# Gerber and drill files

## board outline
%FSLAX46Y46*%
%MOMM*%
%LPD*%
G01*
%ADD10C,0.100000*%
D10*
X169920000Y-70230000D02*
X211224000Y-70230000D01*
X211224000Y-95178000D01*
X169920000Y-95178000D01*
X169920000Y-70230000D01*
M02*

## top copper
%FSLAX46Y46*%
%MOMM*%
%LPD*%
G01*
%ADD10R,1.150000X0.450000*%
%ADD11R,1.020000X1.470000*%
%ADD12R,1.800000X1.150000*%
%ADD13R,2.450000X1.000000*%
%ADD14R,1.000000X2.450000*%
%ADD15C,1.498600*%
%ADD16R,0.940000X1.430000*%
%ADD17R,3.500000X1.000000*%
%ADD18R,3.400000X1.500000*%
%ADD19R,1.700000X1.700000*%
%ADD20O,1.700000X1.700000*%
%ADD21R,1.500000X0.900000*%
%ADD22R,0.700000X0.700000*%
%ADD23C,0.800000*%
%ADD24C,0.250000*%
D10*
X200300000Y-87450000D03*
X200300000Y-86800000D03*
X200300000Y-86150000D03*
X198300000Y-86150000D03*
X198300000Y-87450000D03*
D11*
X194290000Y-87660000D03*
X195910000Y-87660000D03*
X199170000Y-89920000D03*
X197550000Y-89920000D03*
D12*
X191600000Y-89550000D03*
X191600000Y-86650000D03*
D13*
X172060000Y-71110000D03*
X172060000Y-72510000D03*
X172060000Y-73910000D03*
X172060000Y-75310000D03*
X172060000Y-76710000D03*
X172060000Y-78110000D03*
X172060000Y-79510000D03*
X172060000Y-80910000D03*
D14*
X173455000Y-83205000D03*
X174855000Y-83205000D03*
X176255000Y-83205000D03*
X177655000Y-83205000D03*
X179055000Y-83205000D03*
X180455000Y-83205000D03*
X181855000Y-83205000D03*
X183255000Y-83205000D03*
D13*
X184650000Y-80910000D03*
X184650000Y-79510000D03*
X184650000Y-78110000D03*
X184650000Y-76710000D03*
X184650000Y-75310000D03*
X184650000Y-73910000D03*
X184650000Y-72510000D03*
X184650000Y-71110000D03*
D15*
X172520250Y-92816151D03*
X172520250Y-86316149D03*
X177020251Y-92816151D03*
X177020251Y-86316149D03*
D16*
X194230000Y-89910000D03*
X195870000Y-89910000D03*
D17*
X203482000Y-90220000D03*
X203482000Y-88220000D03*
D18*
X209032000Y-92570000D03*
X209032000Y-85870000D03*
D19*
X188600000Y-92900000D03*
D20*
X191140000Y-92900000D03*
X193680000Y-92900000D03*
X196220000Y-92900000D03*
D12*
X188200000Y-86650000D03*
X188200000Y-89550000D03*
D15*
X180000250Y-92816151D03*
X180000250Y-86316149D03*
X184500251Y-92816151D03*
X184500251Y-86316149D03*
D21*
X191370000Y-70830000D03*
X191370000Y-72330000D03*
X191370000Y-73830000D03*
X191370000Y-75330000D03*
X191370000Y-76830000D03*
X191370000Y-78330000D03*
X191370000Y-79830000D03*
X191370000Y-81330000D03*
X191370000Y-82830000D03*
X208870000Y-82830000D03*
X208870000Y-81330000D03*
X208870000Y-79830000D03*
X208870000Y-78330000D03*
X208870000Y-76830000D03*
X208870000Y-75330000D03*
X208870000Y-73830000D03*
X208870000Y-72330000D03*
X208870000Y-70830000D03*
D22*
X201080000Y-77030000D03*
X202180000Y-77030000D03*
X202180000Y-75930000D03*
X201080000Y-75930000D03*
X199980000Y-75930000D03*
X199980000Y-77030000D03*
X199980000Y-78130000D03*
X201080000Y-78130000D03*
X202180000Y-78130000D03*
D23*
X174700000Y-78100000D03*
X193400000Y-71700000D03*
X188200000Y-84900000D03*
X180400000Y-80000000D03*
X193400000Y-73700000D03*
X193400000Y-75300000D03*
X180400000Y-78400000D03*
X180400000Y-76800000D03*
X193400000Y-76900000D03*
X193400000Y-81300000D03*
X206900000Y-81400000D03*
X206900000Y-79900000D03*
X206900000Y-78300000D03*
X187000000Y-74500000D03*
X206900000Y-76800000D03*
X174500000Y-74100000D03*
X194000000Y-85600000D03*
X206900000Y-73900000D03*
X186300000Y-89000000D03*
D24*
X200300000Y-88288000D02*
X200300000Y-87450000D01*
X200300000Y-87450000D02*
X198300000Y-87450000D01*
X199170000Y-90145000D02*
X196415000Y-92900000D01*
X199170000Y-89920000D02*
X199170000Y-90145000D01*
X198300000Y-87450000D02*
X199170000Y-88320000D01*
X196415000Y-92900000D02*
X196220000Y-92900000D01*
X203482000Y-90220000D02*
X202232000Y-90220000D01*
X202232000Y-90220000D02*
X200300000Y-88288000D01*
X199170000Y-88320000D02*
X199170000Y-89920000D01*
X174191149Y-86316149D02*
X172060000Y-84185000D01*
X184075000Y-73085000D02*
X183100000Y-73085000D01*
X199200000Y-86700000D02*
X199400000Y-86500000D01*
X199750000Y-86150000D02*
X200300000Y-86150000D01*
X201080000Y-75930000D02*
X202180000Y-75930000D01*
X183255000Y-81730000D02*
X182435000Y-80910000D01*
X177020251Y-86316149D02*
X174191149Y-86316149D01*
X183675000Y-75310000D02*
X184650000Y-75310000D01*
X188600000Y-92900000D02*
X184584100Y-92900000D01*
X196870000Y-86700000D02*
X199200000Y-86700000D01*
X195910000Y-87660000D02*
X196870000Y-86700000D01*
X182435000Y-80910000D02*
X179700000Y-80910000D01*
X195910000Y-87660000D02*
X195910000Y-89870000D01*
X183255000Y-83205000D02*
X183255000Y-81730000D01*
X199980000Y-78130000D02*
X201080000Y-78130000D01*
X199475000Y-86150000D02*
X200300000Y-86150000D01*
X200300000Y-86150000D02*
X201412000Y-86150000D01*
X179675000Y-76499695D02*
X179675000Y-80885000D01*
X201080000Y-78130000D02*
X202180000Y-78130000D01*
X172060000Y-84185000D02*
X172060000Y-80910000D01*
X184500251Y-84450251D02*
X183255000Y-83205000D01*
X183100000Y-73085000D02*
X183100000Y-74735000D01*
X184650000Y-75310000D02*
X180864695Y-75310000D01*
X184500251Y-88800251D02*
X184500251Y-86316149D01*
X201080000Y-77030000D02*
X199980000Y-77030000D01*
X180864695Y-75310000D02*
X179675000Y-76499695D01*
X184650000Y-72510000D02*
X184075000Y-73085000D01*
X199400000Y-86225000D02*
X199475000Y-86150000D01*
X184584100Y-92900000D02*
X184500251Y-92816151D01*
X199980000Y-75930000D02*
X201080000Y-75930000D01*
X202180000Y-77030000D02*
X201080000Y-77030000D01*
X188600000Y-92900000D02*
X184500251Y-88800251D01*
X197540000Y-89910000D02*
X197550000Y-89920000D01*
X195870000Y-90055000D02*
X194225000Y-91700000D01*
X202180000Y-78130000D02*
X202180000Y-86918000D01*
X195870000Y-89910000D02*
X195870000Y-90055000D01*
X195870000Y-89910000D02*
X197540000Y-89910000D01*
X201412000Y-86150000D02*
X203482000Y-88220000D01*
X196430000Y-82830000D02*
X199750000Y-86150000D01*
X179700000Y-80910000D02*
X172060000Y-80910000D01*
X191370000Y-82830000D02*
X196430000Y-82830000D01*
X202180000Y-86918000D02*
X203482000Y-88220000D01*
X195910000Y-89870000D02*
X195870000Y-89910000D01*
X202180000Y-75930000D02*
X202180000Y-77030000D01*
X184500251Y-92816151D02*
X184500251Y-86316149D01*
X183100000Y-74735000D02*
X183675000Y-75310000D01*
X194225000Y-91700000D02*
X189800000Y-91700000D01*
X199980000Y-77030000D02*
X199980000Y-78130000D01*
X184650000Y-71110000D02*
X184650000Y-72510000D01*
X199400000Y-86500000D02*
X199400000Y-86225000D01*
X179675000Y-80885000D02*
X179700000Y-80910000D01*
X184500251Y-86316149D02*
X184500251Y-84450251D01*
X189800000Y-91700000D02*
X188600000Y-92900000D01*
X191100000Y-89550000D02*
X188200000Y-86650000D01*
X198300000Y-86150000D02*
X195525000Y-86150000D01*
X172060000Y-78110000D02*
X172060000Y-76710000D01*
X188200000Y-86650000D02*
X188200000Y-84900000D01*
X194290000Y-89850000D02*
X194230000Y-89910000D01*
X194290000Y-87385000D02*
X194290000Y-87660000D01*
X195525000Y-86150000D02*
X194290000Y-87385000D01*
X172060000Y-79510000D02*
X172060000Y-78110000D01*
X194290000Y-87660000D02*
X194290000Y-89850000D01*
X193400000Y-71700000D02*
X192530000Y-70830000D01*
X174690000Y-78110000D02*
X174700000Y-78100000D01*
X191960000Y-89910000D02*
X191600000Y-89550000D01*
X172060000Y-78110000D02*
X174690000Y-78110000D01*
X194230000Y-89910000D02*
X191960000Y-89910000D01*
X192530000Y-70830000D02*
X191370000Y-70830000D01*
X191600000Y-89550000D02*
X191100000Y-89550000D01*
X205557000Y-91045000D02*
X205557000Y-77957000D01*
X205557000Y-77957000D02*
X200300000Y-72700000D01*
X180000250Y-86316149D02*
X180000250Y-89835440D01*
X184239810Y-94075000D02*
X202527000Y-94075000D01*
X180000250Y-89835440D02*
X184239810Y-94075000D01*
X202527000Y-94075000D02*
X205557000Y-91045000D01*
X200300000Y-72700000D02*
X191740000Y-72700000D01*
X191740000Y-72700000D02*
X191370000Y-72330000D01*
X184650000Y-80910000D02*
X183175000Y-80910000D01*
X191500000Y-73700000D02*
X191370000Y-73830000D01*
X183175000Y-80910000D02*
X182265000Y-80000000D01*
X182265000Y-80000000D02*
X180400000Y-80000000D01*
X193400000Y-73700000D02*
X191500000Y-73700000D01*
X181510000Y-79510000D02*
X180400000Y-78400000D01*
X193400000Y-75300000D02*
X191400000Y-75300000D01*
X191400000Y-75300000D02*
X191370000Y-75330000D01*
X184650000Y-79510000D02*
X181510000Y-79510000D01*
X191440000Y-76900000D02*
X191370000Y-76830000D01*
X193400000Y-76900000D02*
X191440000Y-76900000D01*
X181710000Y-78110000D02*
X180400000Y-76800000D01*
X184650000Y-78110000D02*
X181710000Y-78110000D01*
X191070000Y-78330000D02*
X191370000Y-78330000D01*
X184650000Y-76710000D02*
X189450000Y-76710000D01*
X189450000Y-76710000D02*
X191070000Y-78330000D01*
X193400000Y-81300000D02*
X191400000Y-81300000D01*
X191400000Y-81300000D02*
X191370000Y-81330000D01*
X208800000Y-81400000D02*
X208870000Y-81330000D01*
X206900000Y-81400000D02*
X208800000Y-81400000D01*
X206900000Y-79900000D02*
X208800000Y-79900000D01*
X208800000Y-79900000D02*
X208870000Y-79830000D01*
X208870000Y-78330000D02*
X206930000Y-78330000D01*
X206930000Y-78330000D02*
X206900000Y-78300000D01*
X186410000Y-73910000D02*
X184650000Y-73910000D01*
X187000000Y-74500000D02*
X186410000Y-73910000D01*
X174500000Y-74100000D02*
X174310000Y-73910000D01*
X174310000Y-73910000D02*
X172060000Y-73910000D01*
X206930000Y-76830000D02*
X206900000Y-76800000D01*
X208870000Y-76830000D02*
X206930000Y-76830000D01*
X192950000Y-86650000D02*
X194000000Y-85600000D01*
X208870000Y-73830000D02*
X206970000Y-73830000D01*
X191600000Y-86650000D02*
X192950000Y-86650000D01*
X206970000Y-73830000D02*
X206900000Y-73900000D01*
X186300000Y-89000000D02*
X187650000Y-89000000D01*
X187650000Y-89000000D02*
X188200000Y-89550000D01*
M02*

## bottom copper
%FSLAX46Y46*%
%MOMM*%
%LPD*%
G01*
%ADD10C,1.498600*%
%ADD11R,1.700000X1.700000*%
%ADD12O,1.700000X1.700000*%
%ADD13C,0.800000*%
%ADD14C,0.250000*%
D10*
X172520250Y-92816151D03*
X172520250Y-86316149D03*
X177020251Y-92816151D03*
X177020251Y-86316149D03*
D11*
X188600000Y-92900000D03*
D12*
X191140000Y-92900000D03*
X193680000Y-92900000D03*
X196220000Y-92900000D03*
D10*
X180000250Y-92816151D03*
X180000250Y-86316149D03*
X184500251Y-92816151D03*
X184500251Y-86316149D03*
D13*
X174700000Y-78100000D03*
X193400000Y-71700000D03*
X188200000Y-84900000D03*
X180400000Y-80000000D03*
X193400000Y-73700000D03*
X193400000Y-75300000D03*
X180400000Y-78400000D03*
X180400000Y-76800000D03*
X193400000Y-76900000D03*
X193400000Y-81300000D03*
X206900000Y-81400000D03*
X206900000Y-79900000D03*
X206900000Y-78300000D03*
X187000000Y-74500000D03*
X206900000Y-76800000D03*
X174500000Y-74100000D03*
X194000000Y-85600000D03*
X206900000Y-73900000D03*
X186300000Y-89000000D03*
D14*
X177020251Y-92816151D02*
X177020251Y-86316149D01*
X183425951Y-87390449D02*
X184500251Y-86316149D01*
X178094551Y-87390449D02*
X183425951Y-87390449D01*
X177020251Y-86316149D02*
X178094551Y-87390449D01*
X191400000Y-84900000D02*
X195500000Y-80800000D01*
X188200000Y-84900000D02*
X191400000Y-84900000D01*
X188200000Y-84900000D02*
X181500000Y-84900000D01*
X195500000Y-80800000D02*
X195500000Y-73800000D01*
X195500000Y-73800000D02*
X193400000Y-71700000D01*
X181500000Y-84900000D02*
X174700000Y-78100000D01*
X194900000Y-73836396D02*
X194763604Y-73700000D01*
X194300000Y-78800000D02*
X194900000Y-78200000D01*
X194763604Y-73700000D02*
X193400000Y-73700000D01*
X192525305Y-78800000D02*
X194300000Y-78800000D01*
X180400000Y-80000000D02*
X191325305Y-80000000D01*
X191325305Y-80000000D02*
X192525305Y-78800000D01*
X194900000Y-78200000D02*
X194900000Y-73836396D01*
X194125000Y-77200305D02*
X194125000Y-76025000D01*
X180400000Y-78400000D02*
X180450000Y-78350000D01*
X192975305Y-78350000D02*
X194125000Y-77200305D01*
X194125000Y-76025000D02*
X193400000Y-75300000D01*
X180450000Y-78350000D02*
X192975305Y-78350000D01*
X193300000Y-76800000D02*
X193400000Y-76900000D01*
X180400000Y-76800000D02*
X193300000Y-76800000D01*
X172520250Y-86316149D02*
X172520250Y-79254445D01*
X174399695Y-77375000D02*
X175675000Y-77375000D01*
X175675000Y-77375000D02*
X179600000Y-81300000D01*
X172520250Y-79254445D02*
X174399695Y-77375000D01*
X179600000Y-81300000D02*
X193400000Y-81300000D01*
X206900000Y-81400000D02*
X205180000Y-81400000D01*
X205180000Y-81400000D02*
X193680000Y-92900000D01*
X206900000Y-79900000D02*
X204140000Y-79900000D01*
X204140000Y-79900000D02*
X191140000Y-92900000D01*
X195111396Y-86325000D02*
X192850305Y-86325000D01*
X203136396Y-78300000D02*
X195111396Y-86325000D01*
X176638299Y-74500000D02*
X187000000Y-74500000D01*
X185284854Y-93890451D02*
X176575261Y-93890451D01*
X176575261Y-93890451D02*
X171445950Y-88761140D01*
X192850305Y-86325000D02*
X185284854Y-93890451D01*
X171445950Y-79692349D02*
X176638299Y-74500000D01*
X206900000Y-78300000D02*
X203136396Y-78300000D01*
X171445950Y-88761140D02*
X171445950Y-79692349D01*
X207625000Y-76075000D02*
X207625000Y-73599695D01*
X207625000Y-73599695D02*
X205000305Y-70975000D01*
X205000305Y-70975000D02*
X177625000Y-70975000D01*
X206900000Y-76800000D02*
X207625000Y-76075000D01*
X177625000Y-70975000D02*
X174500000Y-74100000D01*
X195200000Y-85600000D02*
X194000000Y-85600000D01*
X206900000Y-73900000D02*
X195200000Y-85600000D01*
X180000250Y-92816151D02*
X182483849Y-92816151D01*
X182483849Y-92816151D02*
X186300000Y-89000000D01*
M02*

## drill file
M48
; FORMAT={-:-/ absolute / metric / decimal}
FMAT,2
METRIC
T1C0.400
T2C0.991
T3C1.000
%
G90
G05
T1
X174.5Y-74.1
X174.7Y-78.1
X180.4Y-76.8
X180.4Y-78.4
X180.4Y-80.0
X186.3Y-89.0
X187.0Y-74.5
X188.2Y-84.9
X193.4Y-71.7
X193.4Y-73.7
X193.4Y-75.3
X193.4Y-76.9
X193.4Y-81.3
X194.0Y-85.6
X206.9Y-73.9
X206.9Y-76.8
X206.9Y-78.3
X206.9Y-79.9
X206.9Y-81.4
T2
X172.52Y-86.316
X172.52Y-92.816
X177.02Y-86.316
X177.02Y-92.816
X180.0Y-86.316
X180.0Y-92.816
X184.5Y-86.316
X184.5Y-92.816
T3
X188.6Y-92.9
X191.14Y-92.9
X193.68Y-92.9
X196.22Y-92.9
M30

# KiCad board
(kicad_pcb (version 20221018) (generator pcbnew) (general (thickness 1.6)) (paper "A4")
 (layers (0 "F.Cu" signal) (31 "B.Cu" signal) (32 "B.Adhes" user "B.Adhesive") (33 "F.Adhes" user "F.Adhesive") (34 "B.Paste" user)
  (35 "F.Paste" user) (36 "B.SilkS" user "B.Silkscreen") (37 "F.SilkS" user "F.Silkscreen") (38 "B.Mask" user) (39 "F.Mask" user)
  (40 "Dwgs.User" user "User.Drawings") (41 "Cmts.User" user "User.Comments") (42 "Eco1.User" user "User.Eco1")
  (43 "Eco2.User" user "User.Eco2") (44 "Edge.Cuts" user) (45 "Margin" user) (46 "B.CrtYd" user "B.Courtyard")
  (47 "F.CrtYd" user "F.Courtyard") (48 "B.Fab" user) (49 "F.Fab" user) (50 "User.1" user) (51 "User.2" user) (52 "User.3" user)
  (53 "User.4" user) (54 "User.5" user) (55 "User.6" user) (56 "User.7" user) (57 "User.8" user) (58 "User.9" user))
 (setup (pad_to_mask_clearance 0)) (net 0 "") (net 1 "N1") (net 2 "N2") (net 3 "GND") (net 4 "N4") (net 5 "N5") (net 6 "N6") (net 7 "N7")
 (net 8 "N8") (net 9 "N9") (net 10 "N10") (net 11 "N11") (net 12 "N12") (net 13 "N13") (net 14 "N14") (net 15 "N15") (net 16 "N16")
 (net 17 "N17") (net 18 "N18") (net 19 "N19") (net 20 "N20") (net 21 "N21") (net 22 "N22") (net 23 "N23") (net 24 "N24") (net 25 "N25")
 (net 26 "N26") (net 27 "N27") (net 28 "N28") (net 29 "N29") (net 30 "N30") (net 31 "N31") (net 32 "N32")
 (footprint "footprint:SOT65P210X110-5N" (layer "F.Cu") (at 199.3 86.8 180)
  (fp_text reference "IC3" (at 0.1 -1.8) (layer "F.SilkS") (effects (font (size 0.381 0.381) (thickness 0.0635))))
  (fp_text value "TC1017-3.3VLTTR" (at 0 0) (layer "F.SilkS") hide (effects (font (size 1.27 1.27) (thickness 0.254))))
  (pad "1" smd rect (at -1 -0.65 270) (size 0.45 1.15) (layers "F.Cu" "F.Paste" "F.Mask") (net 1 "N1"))
  (pad "2" smd rect (at -1 0 270) (size 0.45 1.15) (layers "F.Cu" "F.Paste" "F.Mask") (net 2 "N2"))
  (pad "3" smd rect (at -1 0.65 270) (size 0.45 1.15) (layers "F.Cu" "F.Paste" "F.Mask") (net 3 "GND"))
  (pad "4" smd rect (at 1 0.65 270) (size 0.45 1.15) (layers "F.Cu" "F.Paste" "F.Mask") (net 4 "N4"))
  (pad "5" smd rect (at 1 -0.65 270) (size 0.45 1.15) (layers "F.Cu" "F.Paste" "F.Mask") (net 1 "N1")))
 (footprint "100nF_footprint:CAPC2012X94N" (layer "F.Cu") (at 195.1 87.66)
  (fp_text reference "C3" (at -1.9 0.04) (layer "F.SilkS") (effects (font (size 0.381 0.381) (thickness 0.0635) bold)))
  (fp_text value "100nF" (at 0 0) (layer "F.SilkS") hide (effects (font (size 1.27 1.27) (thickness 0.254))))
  (pad "1" smd rect (at -0.81 0) (size 1.02 1.47) (layers "F.Cu" "F.Paste" "F.Mask") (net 4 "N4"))
  (pad "2" smd rect (at 0.81 0) (size 1.02 1.47) (layers "F.Cu" "F.Paste" "F.Mask") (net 3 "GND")))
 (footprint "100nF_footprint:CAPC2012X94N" (layer "F.Cu") (at 198.36 89.92 180)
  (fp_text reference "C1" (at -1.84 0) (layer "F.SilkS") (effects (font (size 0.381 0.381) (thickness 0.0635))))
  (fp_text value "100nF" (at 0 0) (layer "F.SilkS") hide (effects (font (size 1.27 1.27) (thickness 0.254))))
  (pad "1" smd rect (at -0.81 0 180) (size 1.02 1.47) (layers "F.Cu" "F.Paste" "F.Mask") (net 1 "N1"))
  (pad "2" smd rect (at 0.81 0 180) (size 1.02 1.47) (layers "F.Cu" "F.Paste" "F.Mask") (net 3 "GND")))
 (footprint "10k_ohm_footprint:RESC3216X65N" (layer "F.Cu") (at 191.6 88.1 90)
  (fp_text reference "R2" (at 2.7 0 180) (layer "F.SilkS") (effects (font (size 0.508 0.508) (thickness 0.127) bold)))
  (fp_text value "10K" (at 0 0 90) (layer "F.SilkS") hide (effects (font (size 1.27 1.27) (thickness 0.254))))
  (pad "1" smd rect (at -1.45 0 90) (size 1.15 1.8) (layers "F.Cu" "F.Paste" "F.Mask") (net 4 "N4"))
  (pad "2" smd rect (at 1.45 0 90) (size 1.15 1.8) (layers "F.Cu" "F.Paste" "F.Mask") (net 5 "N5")))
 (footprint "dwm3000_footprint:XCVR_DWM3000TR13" (layer "F.Cu") (at 178.355 72.06)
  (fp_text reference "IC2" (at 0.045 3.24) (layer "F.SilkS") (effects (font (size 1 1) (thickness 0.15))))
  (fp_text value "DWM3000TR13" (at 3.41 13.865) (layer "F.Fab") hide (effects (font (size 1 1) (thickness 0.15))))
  (pad "1" smd rect (at -6.295 -0.95) (size 2.45 1) (layers "F.Cu" "F.Paste" "F.Mask") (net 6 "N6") (solder_mask_margin 0.102))
  (pad "2" smd rect (at -6.295 0.45) (size 2.45 1) (layers "F.Cu" "F.Paste" "F.Mask") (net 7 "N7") (solder_mask_margin 0.102))
  (pad "3" smd rect (at -6.295 1.85) (size 2.45 1) (layers "F.Cu" "F.Paste" "F.Mask") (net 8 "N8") (solder_mask_margin 0.102))
  (pad "4" smd rect (at -6.295 3.25) (size 2.45 1) (layers "F.Cu" "F.Paste" "F.Mask") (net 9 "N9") (solder_mask_margin 0.102))
  (pad "5" smd rect (at -6.295 4.65) (size 2.45 1) (layers "F.Cu" "F.Paste" "F.Mask") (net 4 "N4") (solder_mask_margin 0.102))
  (pad "6" smd rect (at -6.295 6.05) (size 2.45 1) (layers "F.Cu" "F.Paste" "F.Mask") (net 4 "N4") (solder_mask_margin 0.102))
  (pad "7" smd rect (at -6.295 7.45) (size 2.45 1) (layers "F.Cu" "F.Paste" "F.Mask") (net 4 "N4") (solder_mask_margin 0.102))
  (pad "8" smd rect (at -6.295 8.85) (size 2.45 1) (layers "F.Cu" "F.Paste" "F.Mask") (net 3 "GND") (solder_mask_margin 0.102))
  (pad "9" smd rect (at -4.9 11.145) (size 1 2.45) (layers "F.Cu" "F.Paste" "F.Mask") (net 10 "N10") (solder_mask_margin 0.102))
  (pad "10" smd rect (at -3.5 11.145) (size 1 2.45) (layers "F.Cu" "F.Paste" "F.Mask") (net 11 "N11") (solder_mask_margin 0.102))
  (pad "11" smd rect (at -2.1 11.145) (size 1 2.45) (layers "F.Cu" "F.Paste" "F.Mask") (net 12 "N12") (solder_mask_margin 0.102))
  (pad "12" smd rect (at -0.7 11.145) (size 1 2.45) (layers "F.Cu" "F.Paste" "F.Mask") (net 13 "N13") (solder_mask_margin 0.102))
  (pad "13" smd rect (at 0.7 11.145) (size 1 2.45) (layers "F.Cu" "F.Paste" "F.Mask") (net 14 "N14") (solder_mask_margin 0.102))
  (pad "14" smd rect (at 2.1 11.145) (size 1 2.45) (layers "F.Cu" "F.Paste" "F.Mask") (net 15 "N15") (solder_mask_margin 0.102))
  (pad "15" smd rect (at 3.5 11.145) (size 1 2.45) (layers "F.Cu" "F.Paste" "F.Mask") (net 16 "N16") (solder_mask_margin 0.102))
  (pad "16" smd rect (at 4.9 11.145) (size 1 2.45) (layers "F.Cu" "F.Paste" "F.Mask") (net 3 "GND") (solder_mask_margin 0.102))
  (pad "17" smd rect (at 6.295 8.85) (size 2.45 1) (layers "F.Cu" "F.Paste" "F.Mask") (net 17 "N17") (solder_mask_margin 0.102))
  (pad "18" smd rect (at 6.295 7.45) (size 2.45 1) (layers "F.Cu" "F.Paste" "F.Mask") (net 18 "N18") (solder_mask_margin 0.102))
  (pad "19" smd rect (at 6.295 6.05) (size 2.45 1) (layers "F.Cu" "F.Paste" "F.Mask") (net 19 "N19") (solder_mask_margin 0.102))
  (pad "20" smd rect (at 6.295 4.65) (size 2.45 1) (layers "F.Cu" "F.Paste" "F.Mask") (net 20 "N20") (solder_mask_margin 0.102))
  (pad "21" smd rect (at 6.295 3.25) (size 2.45 1) (layers "F.Cu" "F.Paste" "F.Mask") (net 3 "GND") (solder_mask_margin 0.102))
  (pad "22" smd rect (at 6.295 1.85) (size 2.45 1) (layers "F.Cu" "F.Paste" "F.Mask") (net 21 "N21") (solder_mask_margin 0.102))
  (pad "23" smd rect (at 6.295 0.45) (size 2.45 1) (layers "F.Cu" "F.Paste" "F.Mask") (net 3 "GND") (solder_mask_margin 0.102))
  (pad "24" smd rect (at 6.295 -0.95) (size 2.45 1) (layers "F.Cu" "F.Paste" "F.Mask") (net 3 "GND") (solder_mask_margin 0.102))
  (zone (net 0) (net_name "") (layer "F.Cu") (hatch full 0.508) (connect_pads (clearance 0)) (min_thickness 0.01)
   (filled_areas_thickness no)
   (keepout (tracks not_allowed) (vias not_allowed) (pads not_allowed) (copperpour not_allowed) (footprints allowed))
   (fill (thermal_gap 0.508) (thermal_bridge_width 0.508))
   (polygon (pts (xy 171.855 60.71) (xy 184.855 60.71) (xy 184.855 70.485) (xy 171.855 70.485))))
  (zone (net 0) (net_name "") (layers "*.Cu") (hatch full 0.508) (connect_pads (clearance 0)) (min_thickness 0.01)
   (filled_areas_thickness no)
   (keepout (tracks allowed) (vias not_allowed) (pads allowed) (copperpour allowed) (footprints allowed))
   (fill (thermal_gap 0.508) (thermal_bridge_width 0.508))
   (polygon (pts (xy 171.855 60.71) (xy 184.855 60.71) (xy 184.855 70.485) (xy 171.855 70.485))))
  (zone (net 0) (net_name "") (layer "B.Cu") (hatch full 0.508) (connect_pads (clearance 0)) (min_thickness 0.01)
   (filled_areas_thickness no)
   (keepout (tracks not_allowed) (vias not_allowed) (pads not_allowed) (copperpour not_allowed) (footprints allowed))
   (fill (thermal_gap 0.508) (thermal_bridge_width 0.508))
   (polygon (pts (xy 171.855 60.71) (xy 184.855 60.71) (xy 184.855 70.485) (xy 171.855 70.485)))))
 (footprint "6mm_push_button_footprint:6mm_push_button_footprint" (layer "F.Cu") (at 172.52025 92.816151 90)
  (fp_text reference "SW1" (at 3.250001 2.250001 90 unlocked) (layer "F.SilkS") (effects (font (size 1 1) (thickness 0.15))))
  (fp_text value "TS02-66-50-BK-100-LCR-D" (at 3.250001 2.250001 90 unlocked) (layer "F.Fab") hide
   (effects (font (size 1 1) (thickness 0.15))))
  (pad "1" thru_hole circle (at 0 0 90) (size 1.4986 1.4986) (drill 0.9906) (layers "*.Cu" "*.Mask") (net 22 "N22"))
  (pad "2" thru_hole circle (at 6.500002 0 90) (size 1.4986 1.4986) (drill 0.9906) (layers "*.Cu" "*.Mask") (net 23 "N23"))
  (pad "3" thru_hole circle (at 0 4.500001 90) (size 1.4986 1.4986) (drill 0.9906) (layers "*.Cu" "*.Mask") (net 3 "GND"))
  (pad "4" thru_hole circle (at 6.500002 4.500001 90) (size 1.4986 1.4986) (drill 0.9906) (layers "*.Cu" "*.Mask") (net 3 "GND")))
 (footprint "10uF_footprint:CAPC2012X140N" (layer "F.Cu") (at 195.05 89.91)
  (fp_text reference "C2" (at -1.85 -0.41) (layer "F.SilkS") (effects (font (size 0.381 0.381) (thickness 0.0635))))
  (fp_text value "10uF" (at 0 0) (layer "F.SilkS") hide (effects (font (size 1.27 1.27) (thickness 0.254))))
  (pad "1" smd rect (at -0.82 0) (size 0.94 1.43) (layers "F.Cu" "F.Paste" "F.Mask") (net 4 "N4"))
  (pad "2" smd rect (at 0.82 0) (size 0.94 1.43) (layers "F.Cu" "F.Paste" "F.Mask") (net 3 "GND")))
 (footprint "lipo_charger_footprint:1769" (layer "F.Cu") (at 203.482 89.22 90)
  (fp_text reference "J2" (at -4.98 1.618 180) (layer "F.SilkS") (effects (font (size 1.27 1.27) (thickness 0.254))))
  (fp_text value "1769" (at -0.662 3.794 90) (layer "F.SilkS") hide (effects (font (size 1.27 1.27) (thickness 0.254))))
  (pad "1" smd rect (at -1 0 90) (size 1 3.5) (layers "F.Cu" "F.Paste" "F.Mask") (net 1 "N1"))
  (pad "2" smd rect (at 1 0 90) (size 1 3.5) (layers "F.Cu" "F.Paste" "F.Mask") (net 3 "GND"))
  (pad "3" smd rect (at -3.35 5.55 90) (size 1.5 3.4) (layers "F.Cu" "F.Paste" "F.Mask"))
  (pad "4" smd rect (at 3.35 5.55 90) (size 1.5 3.4) (layers "F.Cu" "F.Paste" "F.Mask")))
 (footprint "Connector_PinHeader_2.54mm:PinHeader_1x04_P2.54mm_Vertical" (layer "F.Cu") (at 188.6 92.9 90)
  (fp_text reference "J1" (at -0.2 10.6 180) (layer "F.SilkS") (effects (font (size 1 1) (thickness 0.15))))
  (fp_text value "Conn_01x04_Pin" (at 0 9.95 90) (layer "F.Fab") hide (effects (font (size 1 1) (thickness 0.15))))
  (pad "1" thru_hole rect (at 0 0 90) (size 1.7 1.7) (drill 1) (layers "*.Cu" "*.Mask") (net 3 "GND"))
  (pad "2" thru_hole oval (at 0 2.54 90) (size 1.7 1.7) (drill 1) (layers "*.Cu" "*.Mask") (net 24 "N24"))
  (pad "3" thru_hole oval (at 0 5.08 90) (size 1.7 1.7) (drill 1) (layers "*.Cu" "*.Mask") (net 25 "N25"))
  (pad "4" thru_hole oval (at 0 7.62 90) (size 1.7 1.7) (drill 1) (layers "*.Cu" "*.Mask") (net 1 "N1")))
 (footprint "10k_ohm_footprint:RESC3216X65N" (layer "F.Cu") (at 188.2 88.1 -90)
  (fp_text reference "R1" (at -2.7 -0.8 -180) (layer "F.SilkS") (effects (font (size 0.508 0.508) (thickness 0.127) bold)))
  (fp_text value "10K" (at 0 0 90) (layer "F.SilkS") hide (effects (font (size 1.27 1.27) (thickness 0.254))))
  (pad "1" smd rect (at -1.45 0 270) (size 1.15 1.8) (layers "F.Cu" "F.Paste" "F.Mask") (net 4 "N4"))
  (pad "2" smd rect (at 1.45 0 270) (size 1.15 1.8) (layers "F.Cu" "F.Paste" "F.Mask") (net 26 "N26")))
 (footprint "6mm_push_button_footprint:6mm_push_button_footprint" (layer "F.Cu") (at 180.00025 92.816151 90)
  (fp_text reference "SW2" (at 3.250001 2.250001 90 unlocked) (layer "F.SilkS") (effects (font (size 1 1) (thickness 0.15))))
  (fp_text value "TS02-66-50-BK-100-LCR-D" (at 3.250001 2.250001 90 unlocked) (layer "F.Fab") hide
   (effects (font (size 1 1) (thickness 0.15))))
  (pad "1" thru_hole circle (at 0 0 90) (size 1.4986 1.4986) (drill 0.9906) (layers "*.Cu" "*.Mask") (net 26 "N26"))
  (pad "2" thru_hole circle (at 6.500002 0 90) (size 1.4986 1.4986) (drill 0.9906) (layers "*.Cu" "*.Mask") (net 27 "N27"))
  (pad "3" thru_hole circle (at 0 4.500001 90) (size 1.4986 1.4986) (drill 0.9906) (layers "*.Cu" "*.Mask") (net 3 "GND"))
  (pad "4" thru_hole circle (at 6.500002 4.500001 90) (size 1.4986 1.4986) (drill 0.9906) (layers "*.Cu" "*.Mask") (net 3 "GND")))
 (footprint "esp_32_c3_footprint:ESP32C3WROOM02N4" (layer "F.Cu") (at 201.08 77.03)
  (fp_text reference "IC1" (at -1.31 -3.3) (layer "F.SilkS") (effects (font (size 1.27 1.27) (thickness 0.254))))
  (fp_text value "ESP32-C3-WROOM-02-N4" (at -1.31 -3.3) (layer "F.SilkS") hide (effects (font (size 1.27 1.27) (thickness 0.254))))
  (pad "1" smd rect (at -9.71 -6.2 90) (size 0.9 1.5) (layers "F.Cu" "F.Paste" "F.Mask") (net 4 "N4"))
  (pad "2" smd rect (at -9.71 -4.7 90) (size 0.9 1.5) (layers "F.Cu" "F.Paste" "F.Mask") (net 27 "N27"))
  (pad "3" smd rect (at -9.71 -3.2 90) (size 0.9 1.5) (layers "F.Cu" "F.Paste" "F.Mask") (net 17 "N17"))
  (pad "4" smd rect (at -9.71 -1.7 90) (size 0.9 1.5) (layers "F.Cu" "F.Paste" "F.Mask") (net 18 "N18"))
  (pad "5" smd rect (at -9.71 -0.2 90) (size 0.9 1.5) (layers "F.Cu" "F.Paste" "F.Mask") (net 19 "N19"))
  (pad "6" smd rect (at -9.71 1.3 90) (size 0.9 1.5) (layers "F.Cu" "F.Paste" "F.Mask") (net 20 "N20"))
  (pad "7" smd rect (at -9.71 2.8 90) (size 0.9 1.5) (layers "F.Cu" "F.Paste" "F.Mask") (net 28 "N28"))
  (pad "8" smd rect (at -9.71 4.3 90) (size 0.9 1.5) (layers "F.Cu" "F.Paste" "F.Mask") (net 23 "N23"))
  (pad "9" smd rect (at -9.71 5.8 90) (size 0.9 1.5) (layers "F.Cu" "F.Paste" "F.Mask") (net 3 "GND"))
  (pad "10" smd rect (at 7.79 5.8 90) (size 0.9 1.5) (layers "F.Cu" "F.Paste" "F.Mask") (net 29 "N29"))
  (pad "11" smd rect (at 7.79 4.3 90) (size 0.9 1.5) (layers "F.Cu" "F.Paste" "F.Mask") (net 25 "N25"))
  (pad "12" smd rect (at 7.79 2.8 90) (size 0.9 1.5) (layers "F.Cu" "F.Paste" "F.Mask") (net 24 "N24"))
  (pad "13" smd rect (at 7.79 1.3 90) (size 0.9 1.5) (layers "F.Cu" "F.Paste" "F.Mask") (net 21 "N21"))
  (pad "14" smd rect (at 7.79 -0.2 90) (size 0.9 1.5) (layers "F.Cu" "F.Paste" "F.Mask") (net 8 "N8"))
  (pad "15" smd rect (at 7.79 -1.7 90) (size 0.9 1.5) (layers "F.Cu" "F.Paste" "F.Mask") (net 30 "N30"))
  (pad "16" smd rect (at 7.79 -3.2 90) (size 0.9 1.5) (layers "F.Cu" "F.Paste" "F.Mask") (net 5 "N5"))
  (pad "17" smd rect (at 7.79 -4.7 90) (size 0.9 1.5) (layers "F.Cu" "F.Paste" "F.Mask") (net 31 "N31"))
  (pad "18" smd rect (at 7.79 -6.2 90) (size 0.9 1.5) (layers "F.Cu" "F.Paste" "F.Mask") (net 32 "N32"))
  (pad "19" smd rect (at 0 0 90) (size 0.7 0.7) (layers "F.Cu" "F.Paste" "F.Mask") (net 3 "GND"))
  (pad "20" smd rect (at 1.1 0 90) (size 0.7 0.7) (layers "F.Cu" "F.Paste" "F.Mask") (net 3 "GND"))
  (pad "21" smd rect (at 1.1 -1.1 90) (size 0.7 0.7) (layers "F.Cu" "F.Paste" "F.Mask") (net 3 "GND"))
  (pad "22" smd rect (at 0 -1.1 90) (size 0.7 0.7) (layers "F.Cu" "F.Paste" "F.Mask") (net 3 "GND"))
  (pad "23" smd rect (at -1.1 -1.1 90) (size 0.7 0.7) (layers "F.Cu" "F.Paste" "F.Mask") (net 3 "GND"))
  (pad "24" smd rect (at -1.1 0 90) (size 0.7 0.7) (layers "F.Cu" "F.Paste" "F.Mask") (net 3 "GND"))
  (pad "25" smd rect (at -1.1 1.1 90) (size 0.7 0.7) (layers "F.Cu" "F.Paste" "F.Mask") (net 3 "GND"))
  (pad "26" smd rect (at 0 1.1 90) (size 0.7 0.7) (layers "F.Cu" "F.Paste" "F.Mask") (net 3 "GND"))
  (pad "27" smd rect (at 1.1 1.1 90) (size 0.7 0.7) (layers "F.Cu" "F.Paste" "F.Mask") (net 3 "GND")))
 (gr_rect (start 169.92 70.23) (end 211.224 95.178) (stroke (width 0.1) (type default)) (fill none) (layer "Edge.Cuts"))
 (segment (start 200.3 88.288) (end 200.3 87.45) (width 0.25) (layer "F.Cu") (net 1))
 (segment (start 200.3 87.45) (end 198.3 87.45) (width 0.25) (layer "F.Cu") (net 1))
 (segment (start 199.17 90.145) (end 196.415 92.9) (width 0.25) (layer "F.Cu") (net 1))
 (segment (start 199.17 89.92) (end 199.17 90.145) (width 0.25) (layer "F.Cu") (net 1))
 (segment (start 198.3 87.45) (end 199.17 88.32) (width 0.25) (layer "F.Cu") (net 1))
 (segment (start 196.415 92.9) (end 196.22 92.9) (width 0.25) (layer "F.Cu") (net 1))
 (segment (start 203.482 90.22) (end 202.232 90.22) (width 0.25) (layer "F.Cu") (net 1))
 (segment (start 202.232 90.22) (end 200.3 88.288) (width 0.25) (layer "F.Cu") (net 1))
 (segment (start 199.17 88.32) (end 199.17 89.92) (width 0.25) (layer "F.Cu") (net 1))
 (segment (start 174.191149 86.316149) (end 172.06 84.185) (width 0.25) (layer "F.Cu") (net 3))
 (segment (start 184.075 73.085) (end 183.1 73.085) (width 0.25) (layer "F.Cu") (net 3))
 (segment (start 199.2 86.7) (end 199.4 86.5) (width 0.25) (layer "F.Cu") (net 3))
 (segment (start 199.75 86.15) (end 200.3 86.15) (width 0.25) (layer "F.Cu") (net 3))
 (segment (start 201.08 75.93) (end 202.18 75.93) (width 0.25) (layer "F.Cu") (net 3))
 (segment (start 183.255 81.73) (end 182.435 80.91) (width 0.25) (layer "F.Cu") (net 3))
 (segment (start 177.020251 86.316149) (end 174.191149 86.316149) (width 0.25) (layer "F.Cu") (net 3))
 (segment (start 183.675 75.31) (end 184.65 75.31) (width 0.25) (layer "F.Cu") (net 3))
 (segment (start 188.6 92.9) (end 184.5841 92.9) (width 0.25) (layer "F.Cu") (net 3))
 (segment (start 196.87 86.7) (end 199.2 86.7) (width 0.25) (layer "F.Cu") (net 3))
 (segment (start 195.91 87.66) (end 196.87 86.7) (width 0.25) (layer "F.Cu") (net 3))
 (segment (start 182.435 80.91) (end 179.7 80.91) (width 0.25) (layer "F.Cu") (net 3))
 (segment (start 195.91 87.66) (end 195.91 89.87) (width 0.25) (layer "F.Cu") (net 3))
 (segment (start 183.255 83.205) (end 183.255 81.73) (width 0.25) (layer "F.Cu") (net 3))
 (segment (start 199.98 78.13) (end 201.08 78.13) (width 0.25) (layer "F.Cu") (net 3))
 (segment (start 199.475 86.15) (end 200.3 86.15) (width 0.25) (layer "F.Cu") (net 3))
 (segment (start 200.3 86.15) (end 201.412 86.15) (width 0.25) (layer "F.Cu") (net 3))
 (segment (start 179.675 76.499695) (end 179.675 80.885) (width 0.25) (layer "F.Cu") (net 3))
 (segment (start 201.08 78.13) (end 202.18 78.13) (width 0.25) (layer "F.Cu") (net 3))
 (segment (start 172.06 84.185) (end 172.06 80.91) (width 0.25) (layer "F.Cu") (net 3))
 (segment (start 184.500251 84.450251) (end 183.255 83.205) (width 0.25) (layer "F.Cu") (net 3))
 (segment (start 183.1 73.085) (end 183.1 74.735) (width 0.25) (layer "F.Cu") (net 3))
 (segment (start 184.65 75.31) (end 180.864695 75.31) (width 0.25) (layer "F.Cu") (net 3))
 (segment (start 184.500251 88.800251) (end 184.500251 86.316149) (width 0.25) (layer "F.Cu") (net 3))
 (segment (start 201.08 77.03) (end 199.98 77.03) (width 0.25) (layer "F.Cu") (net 3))
 (segment (start 180.864695 75.31) (end 179.675 76.499695) (width 0.25) (layer "F.Cu") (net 3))
 (segment (start 184.65 72.51) (end 184.075 73.085) (width 0.25) (layer "F.Cu") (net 3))
 (segment (start 199.4 86.225) (end 199.475 86.15) (width 0.25) (layer "F.Cu") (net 3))
 (segment (start 184.5841 92.9) (end 184.500251 92.816151) (width 0.25) (layer "F.Cu") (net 3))
 (segment (start 199.98 75.93) (end 201.08 75.93) (width 0.25) (layer "F.Cu") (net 3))
 (segment (start 202.18 77.03) (end 201.08 77.03) (width 0.25) (layer "F.Cu") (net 3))
 (segment (start 188.6 92.9) (end 184.500251 88.800251) (width 0.25) (layer "F.Cu") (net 3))
 (segment (start 197.54 89.91) (end 197.55 89.92) (width 0.25) (layer "F.Cu") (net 3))
 (segment (start 195.87 90.055) (end 194.225 91.7) (width 0.25) (layer "F.Cu") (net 3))
 (segment (start 202.18 78.13) (end 202.18 86.918) (width 0.25) (layer "F.Cu") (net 3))
 (segment (start 195.87 89.91) (end 195.87 90.055) (width 0.25) (layer "F.Cu") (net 3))
 (segment (start 195.87 89.91) (end 197.54 89.91) (width 0.25) (layer "F.Cu") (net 3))
 (segment (start 201.412 86.15) (end 203.482 88.22) (width 0.25) (layer "F.Cu") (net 3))
 (segment (start 196.43 82.83) (end 199.75 86.15) (width 0.25) (layer "F.Cu") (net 3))
 (segment (start 179.7 80.91) (end 172.06 80.91) (width 0.25) (layer "F.Cu") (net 3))
 (segment (start 191.37 82.83) (end 196.43 82.83) (width 0.25) (layer "F.Cu") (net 3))
 (segment (start 202.18 86.918) (end 203.482 88.22) (width 0.25) (layer "F.Cu") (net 3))
 (segment (start 195.91 89.87) (end 195.87 89.91) (width 0.25) (layer "F.Cu") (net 3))
 (segment (start 202.18 75.93) (end 202.18 77.03) (width 0.25) (layer "F.Cu") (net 3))
 (segment (start 184.500251 92.816151) (end 184.500251 86.316149) (width 0.25) (layer "F.Cu") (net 3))
 (segment (start 183.1 74.735) (end 183.675 75.31) (width 0.25) (layer "F.Cu") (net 3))
 (segment (start 194.225 91.7) (end 189.8 91.7) (width 0.25) (layer "F.Cu") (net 3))
 (segment (start 199.98 77.03) (end 199.98 78.13) (width 0.25) (layer "F.Cu") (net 3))
 (segment (start 184.65 71.11) (end 184.65 72.51) (width 0.25) (layer "F.Cu") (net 3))
 (segment (start 199.4 86.5) (end 199.4 86.225) (width 0.25) (layer "F.Cu") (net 3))
 (segment (start 179.675 80.885) (end 179.7 80.91) (width 0.25) (layer "F.Cu") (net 3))
 (segment (start 184.500251 86.316149) (end 184.500251 84.450251) (width 0.25) (layer "F.Cu") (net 3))
 (segment (start 189.8 91.7) (end 188.6 92.9) (width 0.25) (layer "F.Cu") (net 3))
 (segment (start 177.020251 92.816151) (end 177.020251 86.316149) (width 0.25) (layer "B.Cu") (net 3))
 (segment (start 183.425951 87.390449) (end 184.500251 86.316149) (width 0.25) (layer "B.Cu") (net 3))
 (segment (start 178.094551 87.390449) (end 183.425951 87.390449) (width 0.25) (layer "B.Cu") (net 3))
 (segment (start 177.020251 86.316149) (end 178.094551 87.390449) (width 0.25) (layer "B.Cu") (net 3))
 (segment (start 191.1 89.55) (end 188.2 86.65) (width 0.25) (layer "F.Cu") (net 4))
 (segment (start 198.3 86.15) (end 195.525 86.15) (width 0.25) (layer "F.Cu") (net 4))
 (segment (start 172.06 78.11) (end 172.06 76.71) (width 0.25) (layer "F.Cu") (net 4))
 (segment (start 188.2 86.65) (end 188.2 84.9) (width 0.25) (layer "F.Cu") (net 4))
 (segment (start 194.29 89.85) (end 194.23 89.91) (width 0.25) (layer "F.Cu") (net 4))
 (segment (start 194.29 87.385) (end 194.29 87.66) (width 0.25) (layer "F.Cu") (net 4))
 (segment (start 195.525 86.15) (end 194.29 87.385) (width 0.25) (layer "F.Cu") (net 4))
 (segment (start 172.06 79.51) (end 172.06 78.11) (width 0.25) (layer "F.Cu") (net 4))
 (segment (start 194.29 87.66) (end 194.29 89.85) (width 0.25) (layer "F.Cu") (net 4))
 (segment (start 193.4 71.7) (end 192.53 70.83) (width 0.25) (layer "F.Cu") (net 4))
 (segment (start 174.69 78.11) (end 174.7 78.1) (width 0.25) (layer "F.Cu") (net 4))
 (segment (start 191.96 89.91) (end 191.6 89.55) (width 0.25) (layer "F.Cu") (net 4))
 (segment (start 172.06 78.11) (end 174.69 78.11) (width 0.25) (layer "F.Cu") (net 4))
 (segment (start 194.23 89.91) (end 191.96 89.91) (width 0.25) (layer "F.Cu") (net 4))
 (segment (start 192.53 70.83) (end 191.37 70.83) (width 0.25) (layer "F.Cu") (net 4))
 (segment (start 191.6 89.55) (end 191.1 89.55) (width 0.25) (layer "F.Cu") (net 4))
 (via blind (at 174.7 78.1) (size 0.8) (drill 0.4) (layers "F.Cu" "B.Cu") (free) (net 4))
 (via blind (at 193.4 71.7) (size 0.8) (drill 0.4) (layers "F.Cu" "B.Cu") (free) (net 4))
 (via blind (at 188.2 84.9) (size 0.8) (drill 0.4) (layers "F.Cu" "B.Cu") (free) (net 4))
 (segment (start 191.4 84.9) (end 195.5 80.8) (width 0.25) (layer "B.Cu") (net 4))
 (segment (start 188.2 84.9) (end 191.4 84.9) (width 0.25) (layer "B.Cu") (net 4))
 (segment (start 188.2 84.9) (end 181.5 84.9) (width 0.25) (layer "B.Cu") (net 4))
 (segment (start 195.5 80.8) (end 195.5 73.8) (width 0.25) (layer "B.Cu") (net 4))
 (segment (start 195.5 73.8) (end 193.4 71.7) (width 0.25) (layer "B.Cu") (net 4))
 (segment (start 181.5 84.9) (end 174.7 78.1) (width 0.25) (layer "B.Cu") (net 4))
 (segment (start 205.557 91.045) (end 205.557 77.957) (width 0.25) (layer "F.Cu") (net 27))
 (segment (start 205.557 77.957) (end 200.3 72.7) (width 0.25) (layer "F.Cu") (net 27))
 (segment (start 180.00025 86.316149) (end 180.00025 89.83544) (width 0.25) (layer "F.Cu") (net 27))
 (segment (start 184.23981 94.075) (end 202.527 94.075) (width 0.25) (layer "F.Cu") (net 27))
 (segment (start 180.00025 89.83544) (end 184.23981 94.075) (width 0.25) (layer "F.Cu") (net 27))
 (segment (start 202.527 94.075) (end 205.557 91.045) (width 0.25) (layer "F.Cu") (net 27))
 (segment (start 200.3 72.7) (end 191.74 72.7) (width 0.25) (layer "F.Cu") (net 27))
 (segment (start 191.74 72.7) (end 191.37 72.33) (width 0.25) (layer "F.Cu") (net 27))
 (segment (start 184.65 80.91) (end 183.175 80.91) (width 0.25) (layer "F.Cu") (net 17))
 (segment (start 191.5 73.7) (end 191.37 73.83) (width 0.25) (layer "F.Cu") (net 17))
 (segment (start 183.175 80.91) (end 182.265 80) (width 0.25) (layer "F.Cu") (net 17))
 (segment (start 182.265 80) (end 180.4 80) (width 0.25) (layer "F.Cu") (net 17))
 (segment (start 193.4 73.7) (end 191.5 73.7) (width 0.25) (layer "F.Cu") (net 17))
 (via blind (at 180.4 80) (size 0.8) (drill 0.4) (layers "F.Cu" "B.Cu") (free) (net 17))
 (via blind (at 193.4 73.7) (size 0.8) (drill 0.4) (layers "F.Cu" "B.Cu") (free) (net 17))
 (segment (start 194.9 73.836396) (end 194.763604 73.7) (width 0.25) (layer "B.Cu") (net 17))
 (segment (start 194.3 78.8) (end 194.9 78.2) (width 0.25) (layer "B.Cu") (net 17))
 (segment (start 194.763604 73.7) (end 193.4 73.7) (width 0.25) (layer "B.Cu") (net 17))
 (segment (start 192.525305 78.8) (end 194.3 78.8) (width 0.25) (layer "B.Cu") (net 17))
 (segment (start 180.4 80) (end 191.325305 80) (width 0.25) (layer "B.Cu") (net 17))
 (segment (start 191.325305 80) (end 192.525305 78.8) (width 0.25) (layer "B.Cu") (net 17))
 (segment (start 194.9 78.2) (end 194.9 73.836396) (width 0.25) (layer "B.Cu") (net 17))
 (segment (start 181.51 79.51) (end 180.4 78.4) (width 0.25) (layer "F.Cu") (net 18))
 (segment (start 193.4 75.3) (end 191.4 75.3) (width 0.25) (layer "F.Cu") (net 18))
 (segment (start 191.4 75.3) (end 191.37 75.33) (width 0.25) (layer "F.Cu") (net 18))
 (segment (start 184.65 79.51) (end 181.51 79.51) (width 0.25) (layer "F.Cu") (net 18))
 (via blind (at 193.4 75.3) (size 0.8) (drill 0.4) (layers "F.Cu" "B.Cu") (free) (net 18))
 (via blind (at 180.4 78.4) (size 0.8) (drill 0.4) (layers "F.Cu" "B.Cu") (free) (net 18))
 (segment (start 194.125 77.200305) (end 194.125 76.025) (width 0.25) (layer "B.Cu") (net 18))
 (segment (start 180.4 78.4) (end 180.45 78.35) (width 0.25) (layer "B.Cu") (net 18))
 (segment (start 192.975305 78.35) (end 194.125 77.200305) (width 0.25) (layer "B.Cu") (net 18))
 (segment (start 194.125 76.025) (end 193.4 75.3) (width 0.25) (layer "B.Cu") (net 18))
 (segment (start 180.45 78.35) (end 192.975305 78.35) (width 0.25) (layer "B.Cu") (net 18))
 (segment (start 191.44 76.9) (end 191.37 76.83) (width 0.25) (layer "F.Cu") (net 19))
 (segment (start 193.4 76.9) (end 191.44 76.9) (width 0.25) (layer "F.Cu") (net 19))
 (segment (start 181.71 78.11) (end 180.4 76.8) (width 0.25) (layer "F.Cu") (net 19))
 (segment (start 184.65 78.11) (end 181.71 78.11) (width 0.25) (layer "F.Cu") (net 19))
 (via blind (at 180.4 76.8) (size 0.8) (drill 0.4) (layers "F.Cu" "B.Cu") (free) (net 19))
 (via blind (at 193.4 76.9) (size 0.8) (drill 0.4) (layers "F.Cu" "B.Cu") (free) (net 19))
 (segment (start 193.3 76.8) (end 193.4 76.9) (width 0.25) (layer "B.Cu") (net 19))
 (segment (start 180.4 76.8) (end 193.3 76.8) (width 0.25) (layer "B.Cu") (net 19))
 (segment (start 191.07 78.33) (end 191.37 78.33) (width 0.25) (layer "F.Cu") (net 20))
 (segment (start 184.65 76.71) (end 189.45 76.71) (width 0.25) (layer "F.Cu") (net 20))
 (segment (start 189.45 76.71) (end 191.07 78.33) (width 0.25) (layer "F.Cu") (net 20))
 (segment (start 193.4 81.3) (end 191.4 81.3) (width 0.25) (layer "F.Cu") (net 23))
 (segment (start 191.4 81.3) (end 191.37 81.33) (width 0.25) (layer "F.Cu") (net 23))
 (via blind (at 193.4 81.3) (size 0.8) (drill 0.4) (layers "F.Cu" "B.Cu") (free) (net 23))
 (segment (start 172.52025 86.316149) (end 172.52025 79.254445) (width 0.25) (layer "B.Cu") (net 23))
 (segment (start 174.399695 77.375) (end 175.675 77.375) (width 0.25) (layer "B.Cu") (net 23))
 (segment (start 175.675 77.375) (end 179.6 81.3) (width 0.25) (layer "B.Cu") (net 23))
 (segment (start 172.52025 79.254445) (end 174.399695 77.375) (width 0.25) (layer "B.Cu") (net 23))
 (segment (start 179.6 81.3) (end 193.4 81.3) (width 0.25) (layer "B.Cu") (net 23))
 (segment (start 208.8 81.4) (end 208.87 81.33) (width 0.25) (layer "F.Cu") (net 25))
 (segment (start 206.9 81.4) (end 208.8 81.4) (width 0.25) (layer "F.Cu") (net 25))
 (via blind (at 206.9 81.4) (size 0.8) (drill 0.4) (layers "F.Cu" "B.Cu") (free) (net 25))
 (segment (start 206.9 81.4) (end 205.18 81.4) (width 0.25) (layer "B.Cu") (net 25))
 (segment (start 205.18 81.4) (end 193.68 92.9) (width 0.25) (layer "B.Cu") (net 25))
 (segment (start 206.9 79.9) (end 208.8 79.9) (width 0.25) (layer "F.Cu") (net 24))
 (segment (start 208.8 79.9) (end 208.87 79.83) (width 0.25) (layer "F.Cu") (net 24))
 (via blind (at 206.9 79.9) (size 0.8) (drill 0.4) (layers "F.Cu" "B.Cu") (free) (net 24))
 (segment (start 206.9 79.9) (end 204.14 79.9) (width 0.25) (layer "B.Cu") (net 24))
 (segment (start 204.14 79.9) (end 191.14 92.9) (width 0.25) (layer "B.Cu") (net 24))
 (segment (start 208.87 78.33) (end 206.93 78.33) (width 0.25) (layer "F.Cu") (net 21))
 (segment (start 206.93 78.33) (end 206.9 78.3) (width 0.25) (layer "F.Cu") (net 21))
 (segment (start 186.41 73.91) (end 184.65 73.91) (width 0.25) (layer "F.Cu") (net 21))
 (segment (start 187 74.5) (end 186.41 73.91) (width 0.25) (layer "F.Cu") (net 21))
 (via blind (at 206.9 78.3) (size 0.8) (drill 0.4) (layers "F.Cu" "B.Cu") (free) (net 21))
 (via blind (at 187 74.5) (size 0.8) (drill 0.4) (layers "F.Cu" "B.Cu") (free) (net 21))
 (segment (start 195.111396 86.325) (end 192.850305 86.325) (width 0.25) (layer "B.Cu") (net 21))
 (segment (start 203.136396 78.3) (end 195.111396 86.325) (width 0.25) (layer "B.Cu") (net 21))
 (segment (start 176.638299 74.5) (end 187 74.5) (width 0.25) (layer "B.Cu") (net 21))
 (segment (start 185.284854 93.890451) (end 176.575261 93.890451) (width 0.25) (layer "B.Cu") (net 21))
 (segment (start 176.575261 93.890451) (end 171.44595 88.76114) (width 0.25) (layer "B.Cu") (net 21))
 (segment (start 192.850305 86.325) (end 185.284854 93.890451) (width 0.25) (layer "B.Cu") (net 21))
 (segment (start 171.44595 79.692349) (end 176.638299 74.5) (width 0.25) (layer "B.Cu") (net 21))
 (segment (start 206.9 78.3) (end 203.136396 78.3) (width 0.25) (layer "B.Cu") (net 21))
 (segment (start 171.44595 88.76114) (end 171.44595 79.692349) (width 0.25) (layer "B.Cu") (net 21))
 (segment (start 174.5 74.1) (end 174.31 73.91) (width 0.25) (layer "F.Cu") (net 8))
 (segment (start 174.31 73.91) (end 172.06 73.91) (width 0.25) (layer "F.Cu") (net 8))
 (segment (start 206.93 76.83) (end 206.9 76.8) (width 0.25) (layer "F.Cu") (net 8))
 (segment (start 208.87 76.83) (end 206.93 76.83) (width 0.25) (layer "F.Cu") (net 8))
 (via blind (at 206.9 76.8) (size 0.8) (drill 0.4) (layers "F.Cu" "B.Cu") (free) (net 8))
 (via blind (at 174.5 74.1) (size 0.8) (drill 0.4) (layers "F.Cu" "B.Cu") (free) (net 8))
 (segment (start 207.625 76.075) (end 207.625 73.599695) (width 0.25) (layer "B.Cu") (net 8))
 (segment (start 207.625 73.599695) (end 205.000305 70.975) (width 0.25) (layer "B.Cu") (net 8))
 (segment (start 205.000305 70.975) (end 177.625 70.975) (width 0.25) (layer "B.Cu") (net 8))
 (segment (start 206.9 76.8) (end 207.625 76.075) (width 0.25) (layer "B.Cu") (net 8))
 (segment (start 177.625 70.975) (end 174.5 74.1) (width 0.25) (layer "B.Cu") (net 8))
 (segment (start 192.95 86.65) (end 194 85.6) (width 0.25) (layer "F.Cu") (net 5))
 (segment (start 208.87 73.83) (end 206.97 73.83) (width 0.25) (layer "F.Cu") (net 5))
 (segment (start 191.6 86.65) (end 192.95 86.65) (width 0.25) (layer "F.Cu") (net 5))
 (segment (start 206.97 73.83) (end 206.9 73.9) (width 0.25) (layer "F.Cu") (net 5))
 (via blind (at 194 85.6) (size 0.8) (drill 0.4) (layers "F.Cu" "B.Cu") (free) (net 5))
 (via blind (at 206.9 73.9) (size 0.8) (drill 0.4) (layers "F.Cu" "B.Cu") (free) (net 5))
 (segment (start 195.2 85.6) (end 194 85.6) (width 0.25) (layer "B.Cu") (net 5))
 (segment (start 206.9 73.9) (end 195.2 85.6) (width 0.25) (layer "B.Cu") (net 5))
 (segment (start 186.3 89) (end 187.65 89) (width 0.25) (layer "F.Cu") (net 26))
 (segment (start 187.65 89) (end 188.2 89.55) (width 0.25) (layer "F.Cu") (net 26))
 (via blind (at 186.3 89) (size 0.8) (drill 0.4) (layers "F.Cu" "B.Cu") (free) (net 26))
 (segment (start 180.00025 92.816151) (end 182.483849 92.816151) (width 0.25) (layer "B.Cu") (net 26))
 (segment (start 182.483849 92.816151) (end 186.3 89) (width 0.25) (layer "B.Cu") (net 26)))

